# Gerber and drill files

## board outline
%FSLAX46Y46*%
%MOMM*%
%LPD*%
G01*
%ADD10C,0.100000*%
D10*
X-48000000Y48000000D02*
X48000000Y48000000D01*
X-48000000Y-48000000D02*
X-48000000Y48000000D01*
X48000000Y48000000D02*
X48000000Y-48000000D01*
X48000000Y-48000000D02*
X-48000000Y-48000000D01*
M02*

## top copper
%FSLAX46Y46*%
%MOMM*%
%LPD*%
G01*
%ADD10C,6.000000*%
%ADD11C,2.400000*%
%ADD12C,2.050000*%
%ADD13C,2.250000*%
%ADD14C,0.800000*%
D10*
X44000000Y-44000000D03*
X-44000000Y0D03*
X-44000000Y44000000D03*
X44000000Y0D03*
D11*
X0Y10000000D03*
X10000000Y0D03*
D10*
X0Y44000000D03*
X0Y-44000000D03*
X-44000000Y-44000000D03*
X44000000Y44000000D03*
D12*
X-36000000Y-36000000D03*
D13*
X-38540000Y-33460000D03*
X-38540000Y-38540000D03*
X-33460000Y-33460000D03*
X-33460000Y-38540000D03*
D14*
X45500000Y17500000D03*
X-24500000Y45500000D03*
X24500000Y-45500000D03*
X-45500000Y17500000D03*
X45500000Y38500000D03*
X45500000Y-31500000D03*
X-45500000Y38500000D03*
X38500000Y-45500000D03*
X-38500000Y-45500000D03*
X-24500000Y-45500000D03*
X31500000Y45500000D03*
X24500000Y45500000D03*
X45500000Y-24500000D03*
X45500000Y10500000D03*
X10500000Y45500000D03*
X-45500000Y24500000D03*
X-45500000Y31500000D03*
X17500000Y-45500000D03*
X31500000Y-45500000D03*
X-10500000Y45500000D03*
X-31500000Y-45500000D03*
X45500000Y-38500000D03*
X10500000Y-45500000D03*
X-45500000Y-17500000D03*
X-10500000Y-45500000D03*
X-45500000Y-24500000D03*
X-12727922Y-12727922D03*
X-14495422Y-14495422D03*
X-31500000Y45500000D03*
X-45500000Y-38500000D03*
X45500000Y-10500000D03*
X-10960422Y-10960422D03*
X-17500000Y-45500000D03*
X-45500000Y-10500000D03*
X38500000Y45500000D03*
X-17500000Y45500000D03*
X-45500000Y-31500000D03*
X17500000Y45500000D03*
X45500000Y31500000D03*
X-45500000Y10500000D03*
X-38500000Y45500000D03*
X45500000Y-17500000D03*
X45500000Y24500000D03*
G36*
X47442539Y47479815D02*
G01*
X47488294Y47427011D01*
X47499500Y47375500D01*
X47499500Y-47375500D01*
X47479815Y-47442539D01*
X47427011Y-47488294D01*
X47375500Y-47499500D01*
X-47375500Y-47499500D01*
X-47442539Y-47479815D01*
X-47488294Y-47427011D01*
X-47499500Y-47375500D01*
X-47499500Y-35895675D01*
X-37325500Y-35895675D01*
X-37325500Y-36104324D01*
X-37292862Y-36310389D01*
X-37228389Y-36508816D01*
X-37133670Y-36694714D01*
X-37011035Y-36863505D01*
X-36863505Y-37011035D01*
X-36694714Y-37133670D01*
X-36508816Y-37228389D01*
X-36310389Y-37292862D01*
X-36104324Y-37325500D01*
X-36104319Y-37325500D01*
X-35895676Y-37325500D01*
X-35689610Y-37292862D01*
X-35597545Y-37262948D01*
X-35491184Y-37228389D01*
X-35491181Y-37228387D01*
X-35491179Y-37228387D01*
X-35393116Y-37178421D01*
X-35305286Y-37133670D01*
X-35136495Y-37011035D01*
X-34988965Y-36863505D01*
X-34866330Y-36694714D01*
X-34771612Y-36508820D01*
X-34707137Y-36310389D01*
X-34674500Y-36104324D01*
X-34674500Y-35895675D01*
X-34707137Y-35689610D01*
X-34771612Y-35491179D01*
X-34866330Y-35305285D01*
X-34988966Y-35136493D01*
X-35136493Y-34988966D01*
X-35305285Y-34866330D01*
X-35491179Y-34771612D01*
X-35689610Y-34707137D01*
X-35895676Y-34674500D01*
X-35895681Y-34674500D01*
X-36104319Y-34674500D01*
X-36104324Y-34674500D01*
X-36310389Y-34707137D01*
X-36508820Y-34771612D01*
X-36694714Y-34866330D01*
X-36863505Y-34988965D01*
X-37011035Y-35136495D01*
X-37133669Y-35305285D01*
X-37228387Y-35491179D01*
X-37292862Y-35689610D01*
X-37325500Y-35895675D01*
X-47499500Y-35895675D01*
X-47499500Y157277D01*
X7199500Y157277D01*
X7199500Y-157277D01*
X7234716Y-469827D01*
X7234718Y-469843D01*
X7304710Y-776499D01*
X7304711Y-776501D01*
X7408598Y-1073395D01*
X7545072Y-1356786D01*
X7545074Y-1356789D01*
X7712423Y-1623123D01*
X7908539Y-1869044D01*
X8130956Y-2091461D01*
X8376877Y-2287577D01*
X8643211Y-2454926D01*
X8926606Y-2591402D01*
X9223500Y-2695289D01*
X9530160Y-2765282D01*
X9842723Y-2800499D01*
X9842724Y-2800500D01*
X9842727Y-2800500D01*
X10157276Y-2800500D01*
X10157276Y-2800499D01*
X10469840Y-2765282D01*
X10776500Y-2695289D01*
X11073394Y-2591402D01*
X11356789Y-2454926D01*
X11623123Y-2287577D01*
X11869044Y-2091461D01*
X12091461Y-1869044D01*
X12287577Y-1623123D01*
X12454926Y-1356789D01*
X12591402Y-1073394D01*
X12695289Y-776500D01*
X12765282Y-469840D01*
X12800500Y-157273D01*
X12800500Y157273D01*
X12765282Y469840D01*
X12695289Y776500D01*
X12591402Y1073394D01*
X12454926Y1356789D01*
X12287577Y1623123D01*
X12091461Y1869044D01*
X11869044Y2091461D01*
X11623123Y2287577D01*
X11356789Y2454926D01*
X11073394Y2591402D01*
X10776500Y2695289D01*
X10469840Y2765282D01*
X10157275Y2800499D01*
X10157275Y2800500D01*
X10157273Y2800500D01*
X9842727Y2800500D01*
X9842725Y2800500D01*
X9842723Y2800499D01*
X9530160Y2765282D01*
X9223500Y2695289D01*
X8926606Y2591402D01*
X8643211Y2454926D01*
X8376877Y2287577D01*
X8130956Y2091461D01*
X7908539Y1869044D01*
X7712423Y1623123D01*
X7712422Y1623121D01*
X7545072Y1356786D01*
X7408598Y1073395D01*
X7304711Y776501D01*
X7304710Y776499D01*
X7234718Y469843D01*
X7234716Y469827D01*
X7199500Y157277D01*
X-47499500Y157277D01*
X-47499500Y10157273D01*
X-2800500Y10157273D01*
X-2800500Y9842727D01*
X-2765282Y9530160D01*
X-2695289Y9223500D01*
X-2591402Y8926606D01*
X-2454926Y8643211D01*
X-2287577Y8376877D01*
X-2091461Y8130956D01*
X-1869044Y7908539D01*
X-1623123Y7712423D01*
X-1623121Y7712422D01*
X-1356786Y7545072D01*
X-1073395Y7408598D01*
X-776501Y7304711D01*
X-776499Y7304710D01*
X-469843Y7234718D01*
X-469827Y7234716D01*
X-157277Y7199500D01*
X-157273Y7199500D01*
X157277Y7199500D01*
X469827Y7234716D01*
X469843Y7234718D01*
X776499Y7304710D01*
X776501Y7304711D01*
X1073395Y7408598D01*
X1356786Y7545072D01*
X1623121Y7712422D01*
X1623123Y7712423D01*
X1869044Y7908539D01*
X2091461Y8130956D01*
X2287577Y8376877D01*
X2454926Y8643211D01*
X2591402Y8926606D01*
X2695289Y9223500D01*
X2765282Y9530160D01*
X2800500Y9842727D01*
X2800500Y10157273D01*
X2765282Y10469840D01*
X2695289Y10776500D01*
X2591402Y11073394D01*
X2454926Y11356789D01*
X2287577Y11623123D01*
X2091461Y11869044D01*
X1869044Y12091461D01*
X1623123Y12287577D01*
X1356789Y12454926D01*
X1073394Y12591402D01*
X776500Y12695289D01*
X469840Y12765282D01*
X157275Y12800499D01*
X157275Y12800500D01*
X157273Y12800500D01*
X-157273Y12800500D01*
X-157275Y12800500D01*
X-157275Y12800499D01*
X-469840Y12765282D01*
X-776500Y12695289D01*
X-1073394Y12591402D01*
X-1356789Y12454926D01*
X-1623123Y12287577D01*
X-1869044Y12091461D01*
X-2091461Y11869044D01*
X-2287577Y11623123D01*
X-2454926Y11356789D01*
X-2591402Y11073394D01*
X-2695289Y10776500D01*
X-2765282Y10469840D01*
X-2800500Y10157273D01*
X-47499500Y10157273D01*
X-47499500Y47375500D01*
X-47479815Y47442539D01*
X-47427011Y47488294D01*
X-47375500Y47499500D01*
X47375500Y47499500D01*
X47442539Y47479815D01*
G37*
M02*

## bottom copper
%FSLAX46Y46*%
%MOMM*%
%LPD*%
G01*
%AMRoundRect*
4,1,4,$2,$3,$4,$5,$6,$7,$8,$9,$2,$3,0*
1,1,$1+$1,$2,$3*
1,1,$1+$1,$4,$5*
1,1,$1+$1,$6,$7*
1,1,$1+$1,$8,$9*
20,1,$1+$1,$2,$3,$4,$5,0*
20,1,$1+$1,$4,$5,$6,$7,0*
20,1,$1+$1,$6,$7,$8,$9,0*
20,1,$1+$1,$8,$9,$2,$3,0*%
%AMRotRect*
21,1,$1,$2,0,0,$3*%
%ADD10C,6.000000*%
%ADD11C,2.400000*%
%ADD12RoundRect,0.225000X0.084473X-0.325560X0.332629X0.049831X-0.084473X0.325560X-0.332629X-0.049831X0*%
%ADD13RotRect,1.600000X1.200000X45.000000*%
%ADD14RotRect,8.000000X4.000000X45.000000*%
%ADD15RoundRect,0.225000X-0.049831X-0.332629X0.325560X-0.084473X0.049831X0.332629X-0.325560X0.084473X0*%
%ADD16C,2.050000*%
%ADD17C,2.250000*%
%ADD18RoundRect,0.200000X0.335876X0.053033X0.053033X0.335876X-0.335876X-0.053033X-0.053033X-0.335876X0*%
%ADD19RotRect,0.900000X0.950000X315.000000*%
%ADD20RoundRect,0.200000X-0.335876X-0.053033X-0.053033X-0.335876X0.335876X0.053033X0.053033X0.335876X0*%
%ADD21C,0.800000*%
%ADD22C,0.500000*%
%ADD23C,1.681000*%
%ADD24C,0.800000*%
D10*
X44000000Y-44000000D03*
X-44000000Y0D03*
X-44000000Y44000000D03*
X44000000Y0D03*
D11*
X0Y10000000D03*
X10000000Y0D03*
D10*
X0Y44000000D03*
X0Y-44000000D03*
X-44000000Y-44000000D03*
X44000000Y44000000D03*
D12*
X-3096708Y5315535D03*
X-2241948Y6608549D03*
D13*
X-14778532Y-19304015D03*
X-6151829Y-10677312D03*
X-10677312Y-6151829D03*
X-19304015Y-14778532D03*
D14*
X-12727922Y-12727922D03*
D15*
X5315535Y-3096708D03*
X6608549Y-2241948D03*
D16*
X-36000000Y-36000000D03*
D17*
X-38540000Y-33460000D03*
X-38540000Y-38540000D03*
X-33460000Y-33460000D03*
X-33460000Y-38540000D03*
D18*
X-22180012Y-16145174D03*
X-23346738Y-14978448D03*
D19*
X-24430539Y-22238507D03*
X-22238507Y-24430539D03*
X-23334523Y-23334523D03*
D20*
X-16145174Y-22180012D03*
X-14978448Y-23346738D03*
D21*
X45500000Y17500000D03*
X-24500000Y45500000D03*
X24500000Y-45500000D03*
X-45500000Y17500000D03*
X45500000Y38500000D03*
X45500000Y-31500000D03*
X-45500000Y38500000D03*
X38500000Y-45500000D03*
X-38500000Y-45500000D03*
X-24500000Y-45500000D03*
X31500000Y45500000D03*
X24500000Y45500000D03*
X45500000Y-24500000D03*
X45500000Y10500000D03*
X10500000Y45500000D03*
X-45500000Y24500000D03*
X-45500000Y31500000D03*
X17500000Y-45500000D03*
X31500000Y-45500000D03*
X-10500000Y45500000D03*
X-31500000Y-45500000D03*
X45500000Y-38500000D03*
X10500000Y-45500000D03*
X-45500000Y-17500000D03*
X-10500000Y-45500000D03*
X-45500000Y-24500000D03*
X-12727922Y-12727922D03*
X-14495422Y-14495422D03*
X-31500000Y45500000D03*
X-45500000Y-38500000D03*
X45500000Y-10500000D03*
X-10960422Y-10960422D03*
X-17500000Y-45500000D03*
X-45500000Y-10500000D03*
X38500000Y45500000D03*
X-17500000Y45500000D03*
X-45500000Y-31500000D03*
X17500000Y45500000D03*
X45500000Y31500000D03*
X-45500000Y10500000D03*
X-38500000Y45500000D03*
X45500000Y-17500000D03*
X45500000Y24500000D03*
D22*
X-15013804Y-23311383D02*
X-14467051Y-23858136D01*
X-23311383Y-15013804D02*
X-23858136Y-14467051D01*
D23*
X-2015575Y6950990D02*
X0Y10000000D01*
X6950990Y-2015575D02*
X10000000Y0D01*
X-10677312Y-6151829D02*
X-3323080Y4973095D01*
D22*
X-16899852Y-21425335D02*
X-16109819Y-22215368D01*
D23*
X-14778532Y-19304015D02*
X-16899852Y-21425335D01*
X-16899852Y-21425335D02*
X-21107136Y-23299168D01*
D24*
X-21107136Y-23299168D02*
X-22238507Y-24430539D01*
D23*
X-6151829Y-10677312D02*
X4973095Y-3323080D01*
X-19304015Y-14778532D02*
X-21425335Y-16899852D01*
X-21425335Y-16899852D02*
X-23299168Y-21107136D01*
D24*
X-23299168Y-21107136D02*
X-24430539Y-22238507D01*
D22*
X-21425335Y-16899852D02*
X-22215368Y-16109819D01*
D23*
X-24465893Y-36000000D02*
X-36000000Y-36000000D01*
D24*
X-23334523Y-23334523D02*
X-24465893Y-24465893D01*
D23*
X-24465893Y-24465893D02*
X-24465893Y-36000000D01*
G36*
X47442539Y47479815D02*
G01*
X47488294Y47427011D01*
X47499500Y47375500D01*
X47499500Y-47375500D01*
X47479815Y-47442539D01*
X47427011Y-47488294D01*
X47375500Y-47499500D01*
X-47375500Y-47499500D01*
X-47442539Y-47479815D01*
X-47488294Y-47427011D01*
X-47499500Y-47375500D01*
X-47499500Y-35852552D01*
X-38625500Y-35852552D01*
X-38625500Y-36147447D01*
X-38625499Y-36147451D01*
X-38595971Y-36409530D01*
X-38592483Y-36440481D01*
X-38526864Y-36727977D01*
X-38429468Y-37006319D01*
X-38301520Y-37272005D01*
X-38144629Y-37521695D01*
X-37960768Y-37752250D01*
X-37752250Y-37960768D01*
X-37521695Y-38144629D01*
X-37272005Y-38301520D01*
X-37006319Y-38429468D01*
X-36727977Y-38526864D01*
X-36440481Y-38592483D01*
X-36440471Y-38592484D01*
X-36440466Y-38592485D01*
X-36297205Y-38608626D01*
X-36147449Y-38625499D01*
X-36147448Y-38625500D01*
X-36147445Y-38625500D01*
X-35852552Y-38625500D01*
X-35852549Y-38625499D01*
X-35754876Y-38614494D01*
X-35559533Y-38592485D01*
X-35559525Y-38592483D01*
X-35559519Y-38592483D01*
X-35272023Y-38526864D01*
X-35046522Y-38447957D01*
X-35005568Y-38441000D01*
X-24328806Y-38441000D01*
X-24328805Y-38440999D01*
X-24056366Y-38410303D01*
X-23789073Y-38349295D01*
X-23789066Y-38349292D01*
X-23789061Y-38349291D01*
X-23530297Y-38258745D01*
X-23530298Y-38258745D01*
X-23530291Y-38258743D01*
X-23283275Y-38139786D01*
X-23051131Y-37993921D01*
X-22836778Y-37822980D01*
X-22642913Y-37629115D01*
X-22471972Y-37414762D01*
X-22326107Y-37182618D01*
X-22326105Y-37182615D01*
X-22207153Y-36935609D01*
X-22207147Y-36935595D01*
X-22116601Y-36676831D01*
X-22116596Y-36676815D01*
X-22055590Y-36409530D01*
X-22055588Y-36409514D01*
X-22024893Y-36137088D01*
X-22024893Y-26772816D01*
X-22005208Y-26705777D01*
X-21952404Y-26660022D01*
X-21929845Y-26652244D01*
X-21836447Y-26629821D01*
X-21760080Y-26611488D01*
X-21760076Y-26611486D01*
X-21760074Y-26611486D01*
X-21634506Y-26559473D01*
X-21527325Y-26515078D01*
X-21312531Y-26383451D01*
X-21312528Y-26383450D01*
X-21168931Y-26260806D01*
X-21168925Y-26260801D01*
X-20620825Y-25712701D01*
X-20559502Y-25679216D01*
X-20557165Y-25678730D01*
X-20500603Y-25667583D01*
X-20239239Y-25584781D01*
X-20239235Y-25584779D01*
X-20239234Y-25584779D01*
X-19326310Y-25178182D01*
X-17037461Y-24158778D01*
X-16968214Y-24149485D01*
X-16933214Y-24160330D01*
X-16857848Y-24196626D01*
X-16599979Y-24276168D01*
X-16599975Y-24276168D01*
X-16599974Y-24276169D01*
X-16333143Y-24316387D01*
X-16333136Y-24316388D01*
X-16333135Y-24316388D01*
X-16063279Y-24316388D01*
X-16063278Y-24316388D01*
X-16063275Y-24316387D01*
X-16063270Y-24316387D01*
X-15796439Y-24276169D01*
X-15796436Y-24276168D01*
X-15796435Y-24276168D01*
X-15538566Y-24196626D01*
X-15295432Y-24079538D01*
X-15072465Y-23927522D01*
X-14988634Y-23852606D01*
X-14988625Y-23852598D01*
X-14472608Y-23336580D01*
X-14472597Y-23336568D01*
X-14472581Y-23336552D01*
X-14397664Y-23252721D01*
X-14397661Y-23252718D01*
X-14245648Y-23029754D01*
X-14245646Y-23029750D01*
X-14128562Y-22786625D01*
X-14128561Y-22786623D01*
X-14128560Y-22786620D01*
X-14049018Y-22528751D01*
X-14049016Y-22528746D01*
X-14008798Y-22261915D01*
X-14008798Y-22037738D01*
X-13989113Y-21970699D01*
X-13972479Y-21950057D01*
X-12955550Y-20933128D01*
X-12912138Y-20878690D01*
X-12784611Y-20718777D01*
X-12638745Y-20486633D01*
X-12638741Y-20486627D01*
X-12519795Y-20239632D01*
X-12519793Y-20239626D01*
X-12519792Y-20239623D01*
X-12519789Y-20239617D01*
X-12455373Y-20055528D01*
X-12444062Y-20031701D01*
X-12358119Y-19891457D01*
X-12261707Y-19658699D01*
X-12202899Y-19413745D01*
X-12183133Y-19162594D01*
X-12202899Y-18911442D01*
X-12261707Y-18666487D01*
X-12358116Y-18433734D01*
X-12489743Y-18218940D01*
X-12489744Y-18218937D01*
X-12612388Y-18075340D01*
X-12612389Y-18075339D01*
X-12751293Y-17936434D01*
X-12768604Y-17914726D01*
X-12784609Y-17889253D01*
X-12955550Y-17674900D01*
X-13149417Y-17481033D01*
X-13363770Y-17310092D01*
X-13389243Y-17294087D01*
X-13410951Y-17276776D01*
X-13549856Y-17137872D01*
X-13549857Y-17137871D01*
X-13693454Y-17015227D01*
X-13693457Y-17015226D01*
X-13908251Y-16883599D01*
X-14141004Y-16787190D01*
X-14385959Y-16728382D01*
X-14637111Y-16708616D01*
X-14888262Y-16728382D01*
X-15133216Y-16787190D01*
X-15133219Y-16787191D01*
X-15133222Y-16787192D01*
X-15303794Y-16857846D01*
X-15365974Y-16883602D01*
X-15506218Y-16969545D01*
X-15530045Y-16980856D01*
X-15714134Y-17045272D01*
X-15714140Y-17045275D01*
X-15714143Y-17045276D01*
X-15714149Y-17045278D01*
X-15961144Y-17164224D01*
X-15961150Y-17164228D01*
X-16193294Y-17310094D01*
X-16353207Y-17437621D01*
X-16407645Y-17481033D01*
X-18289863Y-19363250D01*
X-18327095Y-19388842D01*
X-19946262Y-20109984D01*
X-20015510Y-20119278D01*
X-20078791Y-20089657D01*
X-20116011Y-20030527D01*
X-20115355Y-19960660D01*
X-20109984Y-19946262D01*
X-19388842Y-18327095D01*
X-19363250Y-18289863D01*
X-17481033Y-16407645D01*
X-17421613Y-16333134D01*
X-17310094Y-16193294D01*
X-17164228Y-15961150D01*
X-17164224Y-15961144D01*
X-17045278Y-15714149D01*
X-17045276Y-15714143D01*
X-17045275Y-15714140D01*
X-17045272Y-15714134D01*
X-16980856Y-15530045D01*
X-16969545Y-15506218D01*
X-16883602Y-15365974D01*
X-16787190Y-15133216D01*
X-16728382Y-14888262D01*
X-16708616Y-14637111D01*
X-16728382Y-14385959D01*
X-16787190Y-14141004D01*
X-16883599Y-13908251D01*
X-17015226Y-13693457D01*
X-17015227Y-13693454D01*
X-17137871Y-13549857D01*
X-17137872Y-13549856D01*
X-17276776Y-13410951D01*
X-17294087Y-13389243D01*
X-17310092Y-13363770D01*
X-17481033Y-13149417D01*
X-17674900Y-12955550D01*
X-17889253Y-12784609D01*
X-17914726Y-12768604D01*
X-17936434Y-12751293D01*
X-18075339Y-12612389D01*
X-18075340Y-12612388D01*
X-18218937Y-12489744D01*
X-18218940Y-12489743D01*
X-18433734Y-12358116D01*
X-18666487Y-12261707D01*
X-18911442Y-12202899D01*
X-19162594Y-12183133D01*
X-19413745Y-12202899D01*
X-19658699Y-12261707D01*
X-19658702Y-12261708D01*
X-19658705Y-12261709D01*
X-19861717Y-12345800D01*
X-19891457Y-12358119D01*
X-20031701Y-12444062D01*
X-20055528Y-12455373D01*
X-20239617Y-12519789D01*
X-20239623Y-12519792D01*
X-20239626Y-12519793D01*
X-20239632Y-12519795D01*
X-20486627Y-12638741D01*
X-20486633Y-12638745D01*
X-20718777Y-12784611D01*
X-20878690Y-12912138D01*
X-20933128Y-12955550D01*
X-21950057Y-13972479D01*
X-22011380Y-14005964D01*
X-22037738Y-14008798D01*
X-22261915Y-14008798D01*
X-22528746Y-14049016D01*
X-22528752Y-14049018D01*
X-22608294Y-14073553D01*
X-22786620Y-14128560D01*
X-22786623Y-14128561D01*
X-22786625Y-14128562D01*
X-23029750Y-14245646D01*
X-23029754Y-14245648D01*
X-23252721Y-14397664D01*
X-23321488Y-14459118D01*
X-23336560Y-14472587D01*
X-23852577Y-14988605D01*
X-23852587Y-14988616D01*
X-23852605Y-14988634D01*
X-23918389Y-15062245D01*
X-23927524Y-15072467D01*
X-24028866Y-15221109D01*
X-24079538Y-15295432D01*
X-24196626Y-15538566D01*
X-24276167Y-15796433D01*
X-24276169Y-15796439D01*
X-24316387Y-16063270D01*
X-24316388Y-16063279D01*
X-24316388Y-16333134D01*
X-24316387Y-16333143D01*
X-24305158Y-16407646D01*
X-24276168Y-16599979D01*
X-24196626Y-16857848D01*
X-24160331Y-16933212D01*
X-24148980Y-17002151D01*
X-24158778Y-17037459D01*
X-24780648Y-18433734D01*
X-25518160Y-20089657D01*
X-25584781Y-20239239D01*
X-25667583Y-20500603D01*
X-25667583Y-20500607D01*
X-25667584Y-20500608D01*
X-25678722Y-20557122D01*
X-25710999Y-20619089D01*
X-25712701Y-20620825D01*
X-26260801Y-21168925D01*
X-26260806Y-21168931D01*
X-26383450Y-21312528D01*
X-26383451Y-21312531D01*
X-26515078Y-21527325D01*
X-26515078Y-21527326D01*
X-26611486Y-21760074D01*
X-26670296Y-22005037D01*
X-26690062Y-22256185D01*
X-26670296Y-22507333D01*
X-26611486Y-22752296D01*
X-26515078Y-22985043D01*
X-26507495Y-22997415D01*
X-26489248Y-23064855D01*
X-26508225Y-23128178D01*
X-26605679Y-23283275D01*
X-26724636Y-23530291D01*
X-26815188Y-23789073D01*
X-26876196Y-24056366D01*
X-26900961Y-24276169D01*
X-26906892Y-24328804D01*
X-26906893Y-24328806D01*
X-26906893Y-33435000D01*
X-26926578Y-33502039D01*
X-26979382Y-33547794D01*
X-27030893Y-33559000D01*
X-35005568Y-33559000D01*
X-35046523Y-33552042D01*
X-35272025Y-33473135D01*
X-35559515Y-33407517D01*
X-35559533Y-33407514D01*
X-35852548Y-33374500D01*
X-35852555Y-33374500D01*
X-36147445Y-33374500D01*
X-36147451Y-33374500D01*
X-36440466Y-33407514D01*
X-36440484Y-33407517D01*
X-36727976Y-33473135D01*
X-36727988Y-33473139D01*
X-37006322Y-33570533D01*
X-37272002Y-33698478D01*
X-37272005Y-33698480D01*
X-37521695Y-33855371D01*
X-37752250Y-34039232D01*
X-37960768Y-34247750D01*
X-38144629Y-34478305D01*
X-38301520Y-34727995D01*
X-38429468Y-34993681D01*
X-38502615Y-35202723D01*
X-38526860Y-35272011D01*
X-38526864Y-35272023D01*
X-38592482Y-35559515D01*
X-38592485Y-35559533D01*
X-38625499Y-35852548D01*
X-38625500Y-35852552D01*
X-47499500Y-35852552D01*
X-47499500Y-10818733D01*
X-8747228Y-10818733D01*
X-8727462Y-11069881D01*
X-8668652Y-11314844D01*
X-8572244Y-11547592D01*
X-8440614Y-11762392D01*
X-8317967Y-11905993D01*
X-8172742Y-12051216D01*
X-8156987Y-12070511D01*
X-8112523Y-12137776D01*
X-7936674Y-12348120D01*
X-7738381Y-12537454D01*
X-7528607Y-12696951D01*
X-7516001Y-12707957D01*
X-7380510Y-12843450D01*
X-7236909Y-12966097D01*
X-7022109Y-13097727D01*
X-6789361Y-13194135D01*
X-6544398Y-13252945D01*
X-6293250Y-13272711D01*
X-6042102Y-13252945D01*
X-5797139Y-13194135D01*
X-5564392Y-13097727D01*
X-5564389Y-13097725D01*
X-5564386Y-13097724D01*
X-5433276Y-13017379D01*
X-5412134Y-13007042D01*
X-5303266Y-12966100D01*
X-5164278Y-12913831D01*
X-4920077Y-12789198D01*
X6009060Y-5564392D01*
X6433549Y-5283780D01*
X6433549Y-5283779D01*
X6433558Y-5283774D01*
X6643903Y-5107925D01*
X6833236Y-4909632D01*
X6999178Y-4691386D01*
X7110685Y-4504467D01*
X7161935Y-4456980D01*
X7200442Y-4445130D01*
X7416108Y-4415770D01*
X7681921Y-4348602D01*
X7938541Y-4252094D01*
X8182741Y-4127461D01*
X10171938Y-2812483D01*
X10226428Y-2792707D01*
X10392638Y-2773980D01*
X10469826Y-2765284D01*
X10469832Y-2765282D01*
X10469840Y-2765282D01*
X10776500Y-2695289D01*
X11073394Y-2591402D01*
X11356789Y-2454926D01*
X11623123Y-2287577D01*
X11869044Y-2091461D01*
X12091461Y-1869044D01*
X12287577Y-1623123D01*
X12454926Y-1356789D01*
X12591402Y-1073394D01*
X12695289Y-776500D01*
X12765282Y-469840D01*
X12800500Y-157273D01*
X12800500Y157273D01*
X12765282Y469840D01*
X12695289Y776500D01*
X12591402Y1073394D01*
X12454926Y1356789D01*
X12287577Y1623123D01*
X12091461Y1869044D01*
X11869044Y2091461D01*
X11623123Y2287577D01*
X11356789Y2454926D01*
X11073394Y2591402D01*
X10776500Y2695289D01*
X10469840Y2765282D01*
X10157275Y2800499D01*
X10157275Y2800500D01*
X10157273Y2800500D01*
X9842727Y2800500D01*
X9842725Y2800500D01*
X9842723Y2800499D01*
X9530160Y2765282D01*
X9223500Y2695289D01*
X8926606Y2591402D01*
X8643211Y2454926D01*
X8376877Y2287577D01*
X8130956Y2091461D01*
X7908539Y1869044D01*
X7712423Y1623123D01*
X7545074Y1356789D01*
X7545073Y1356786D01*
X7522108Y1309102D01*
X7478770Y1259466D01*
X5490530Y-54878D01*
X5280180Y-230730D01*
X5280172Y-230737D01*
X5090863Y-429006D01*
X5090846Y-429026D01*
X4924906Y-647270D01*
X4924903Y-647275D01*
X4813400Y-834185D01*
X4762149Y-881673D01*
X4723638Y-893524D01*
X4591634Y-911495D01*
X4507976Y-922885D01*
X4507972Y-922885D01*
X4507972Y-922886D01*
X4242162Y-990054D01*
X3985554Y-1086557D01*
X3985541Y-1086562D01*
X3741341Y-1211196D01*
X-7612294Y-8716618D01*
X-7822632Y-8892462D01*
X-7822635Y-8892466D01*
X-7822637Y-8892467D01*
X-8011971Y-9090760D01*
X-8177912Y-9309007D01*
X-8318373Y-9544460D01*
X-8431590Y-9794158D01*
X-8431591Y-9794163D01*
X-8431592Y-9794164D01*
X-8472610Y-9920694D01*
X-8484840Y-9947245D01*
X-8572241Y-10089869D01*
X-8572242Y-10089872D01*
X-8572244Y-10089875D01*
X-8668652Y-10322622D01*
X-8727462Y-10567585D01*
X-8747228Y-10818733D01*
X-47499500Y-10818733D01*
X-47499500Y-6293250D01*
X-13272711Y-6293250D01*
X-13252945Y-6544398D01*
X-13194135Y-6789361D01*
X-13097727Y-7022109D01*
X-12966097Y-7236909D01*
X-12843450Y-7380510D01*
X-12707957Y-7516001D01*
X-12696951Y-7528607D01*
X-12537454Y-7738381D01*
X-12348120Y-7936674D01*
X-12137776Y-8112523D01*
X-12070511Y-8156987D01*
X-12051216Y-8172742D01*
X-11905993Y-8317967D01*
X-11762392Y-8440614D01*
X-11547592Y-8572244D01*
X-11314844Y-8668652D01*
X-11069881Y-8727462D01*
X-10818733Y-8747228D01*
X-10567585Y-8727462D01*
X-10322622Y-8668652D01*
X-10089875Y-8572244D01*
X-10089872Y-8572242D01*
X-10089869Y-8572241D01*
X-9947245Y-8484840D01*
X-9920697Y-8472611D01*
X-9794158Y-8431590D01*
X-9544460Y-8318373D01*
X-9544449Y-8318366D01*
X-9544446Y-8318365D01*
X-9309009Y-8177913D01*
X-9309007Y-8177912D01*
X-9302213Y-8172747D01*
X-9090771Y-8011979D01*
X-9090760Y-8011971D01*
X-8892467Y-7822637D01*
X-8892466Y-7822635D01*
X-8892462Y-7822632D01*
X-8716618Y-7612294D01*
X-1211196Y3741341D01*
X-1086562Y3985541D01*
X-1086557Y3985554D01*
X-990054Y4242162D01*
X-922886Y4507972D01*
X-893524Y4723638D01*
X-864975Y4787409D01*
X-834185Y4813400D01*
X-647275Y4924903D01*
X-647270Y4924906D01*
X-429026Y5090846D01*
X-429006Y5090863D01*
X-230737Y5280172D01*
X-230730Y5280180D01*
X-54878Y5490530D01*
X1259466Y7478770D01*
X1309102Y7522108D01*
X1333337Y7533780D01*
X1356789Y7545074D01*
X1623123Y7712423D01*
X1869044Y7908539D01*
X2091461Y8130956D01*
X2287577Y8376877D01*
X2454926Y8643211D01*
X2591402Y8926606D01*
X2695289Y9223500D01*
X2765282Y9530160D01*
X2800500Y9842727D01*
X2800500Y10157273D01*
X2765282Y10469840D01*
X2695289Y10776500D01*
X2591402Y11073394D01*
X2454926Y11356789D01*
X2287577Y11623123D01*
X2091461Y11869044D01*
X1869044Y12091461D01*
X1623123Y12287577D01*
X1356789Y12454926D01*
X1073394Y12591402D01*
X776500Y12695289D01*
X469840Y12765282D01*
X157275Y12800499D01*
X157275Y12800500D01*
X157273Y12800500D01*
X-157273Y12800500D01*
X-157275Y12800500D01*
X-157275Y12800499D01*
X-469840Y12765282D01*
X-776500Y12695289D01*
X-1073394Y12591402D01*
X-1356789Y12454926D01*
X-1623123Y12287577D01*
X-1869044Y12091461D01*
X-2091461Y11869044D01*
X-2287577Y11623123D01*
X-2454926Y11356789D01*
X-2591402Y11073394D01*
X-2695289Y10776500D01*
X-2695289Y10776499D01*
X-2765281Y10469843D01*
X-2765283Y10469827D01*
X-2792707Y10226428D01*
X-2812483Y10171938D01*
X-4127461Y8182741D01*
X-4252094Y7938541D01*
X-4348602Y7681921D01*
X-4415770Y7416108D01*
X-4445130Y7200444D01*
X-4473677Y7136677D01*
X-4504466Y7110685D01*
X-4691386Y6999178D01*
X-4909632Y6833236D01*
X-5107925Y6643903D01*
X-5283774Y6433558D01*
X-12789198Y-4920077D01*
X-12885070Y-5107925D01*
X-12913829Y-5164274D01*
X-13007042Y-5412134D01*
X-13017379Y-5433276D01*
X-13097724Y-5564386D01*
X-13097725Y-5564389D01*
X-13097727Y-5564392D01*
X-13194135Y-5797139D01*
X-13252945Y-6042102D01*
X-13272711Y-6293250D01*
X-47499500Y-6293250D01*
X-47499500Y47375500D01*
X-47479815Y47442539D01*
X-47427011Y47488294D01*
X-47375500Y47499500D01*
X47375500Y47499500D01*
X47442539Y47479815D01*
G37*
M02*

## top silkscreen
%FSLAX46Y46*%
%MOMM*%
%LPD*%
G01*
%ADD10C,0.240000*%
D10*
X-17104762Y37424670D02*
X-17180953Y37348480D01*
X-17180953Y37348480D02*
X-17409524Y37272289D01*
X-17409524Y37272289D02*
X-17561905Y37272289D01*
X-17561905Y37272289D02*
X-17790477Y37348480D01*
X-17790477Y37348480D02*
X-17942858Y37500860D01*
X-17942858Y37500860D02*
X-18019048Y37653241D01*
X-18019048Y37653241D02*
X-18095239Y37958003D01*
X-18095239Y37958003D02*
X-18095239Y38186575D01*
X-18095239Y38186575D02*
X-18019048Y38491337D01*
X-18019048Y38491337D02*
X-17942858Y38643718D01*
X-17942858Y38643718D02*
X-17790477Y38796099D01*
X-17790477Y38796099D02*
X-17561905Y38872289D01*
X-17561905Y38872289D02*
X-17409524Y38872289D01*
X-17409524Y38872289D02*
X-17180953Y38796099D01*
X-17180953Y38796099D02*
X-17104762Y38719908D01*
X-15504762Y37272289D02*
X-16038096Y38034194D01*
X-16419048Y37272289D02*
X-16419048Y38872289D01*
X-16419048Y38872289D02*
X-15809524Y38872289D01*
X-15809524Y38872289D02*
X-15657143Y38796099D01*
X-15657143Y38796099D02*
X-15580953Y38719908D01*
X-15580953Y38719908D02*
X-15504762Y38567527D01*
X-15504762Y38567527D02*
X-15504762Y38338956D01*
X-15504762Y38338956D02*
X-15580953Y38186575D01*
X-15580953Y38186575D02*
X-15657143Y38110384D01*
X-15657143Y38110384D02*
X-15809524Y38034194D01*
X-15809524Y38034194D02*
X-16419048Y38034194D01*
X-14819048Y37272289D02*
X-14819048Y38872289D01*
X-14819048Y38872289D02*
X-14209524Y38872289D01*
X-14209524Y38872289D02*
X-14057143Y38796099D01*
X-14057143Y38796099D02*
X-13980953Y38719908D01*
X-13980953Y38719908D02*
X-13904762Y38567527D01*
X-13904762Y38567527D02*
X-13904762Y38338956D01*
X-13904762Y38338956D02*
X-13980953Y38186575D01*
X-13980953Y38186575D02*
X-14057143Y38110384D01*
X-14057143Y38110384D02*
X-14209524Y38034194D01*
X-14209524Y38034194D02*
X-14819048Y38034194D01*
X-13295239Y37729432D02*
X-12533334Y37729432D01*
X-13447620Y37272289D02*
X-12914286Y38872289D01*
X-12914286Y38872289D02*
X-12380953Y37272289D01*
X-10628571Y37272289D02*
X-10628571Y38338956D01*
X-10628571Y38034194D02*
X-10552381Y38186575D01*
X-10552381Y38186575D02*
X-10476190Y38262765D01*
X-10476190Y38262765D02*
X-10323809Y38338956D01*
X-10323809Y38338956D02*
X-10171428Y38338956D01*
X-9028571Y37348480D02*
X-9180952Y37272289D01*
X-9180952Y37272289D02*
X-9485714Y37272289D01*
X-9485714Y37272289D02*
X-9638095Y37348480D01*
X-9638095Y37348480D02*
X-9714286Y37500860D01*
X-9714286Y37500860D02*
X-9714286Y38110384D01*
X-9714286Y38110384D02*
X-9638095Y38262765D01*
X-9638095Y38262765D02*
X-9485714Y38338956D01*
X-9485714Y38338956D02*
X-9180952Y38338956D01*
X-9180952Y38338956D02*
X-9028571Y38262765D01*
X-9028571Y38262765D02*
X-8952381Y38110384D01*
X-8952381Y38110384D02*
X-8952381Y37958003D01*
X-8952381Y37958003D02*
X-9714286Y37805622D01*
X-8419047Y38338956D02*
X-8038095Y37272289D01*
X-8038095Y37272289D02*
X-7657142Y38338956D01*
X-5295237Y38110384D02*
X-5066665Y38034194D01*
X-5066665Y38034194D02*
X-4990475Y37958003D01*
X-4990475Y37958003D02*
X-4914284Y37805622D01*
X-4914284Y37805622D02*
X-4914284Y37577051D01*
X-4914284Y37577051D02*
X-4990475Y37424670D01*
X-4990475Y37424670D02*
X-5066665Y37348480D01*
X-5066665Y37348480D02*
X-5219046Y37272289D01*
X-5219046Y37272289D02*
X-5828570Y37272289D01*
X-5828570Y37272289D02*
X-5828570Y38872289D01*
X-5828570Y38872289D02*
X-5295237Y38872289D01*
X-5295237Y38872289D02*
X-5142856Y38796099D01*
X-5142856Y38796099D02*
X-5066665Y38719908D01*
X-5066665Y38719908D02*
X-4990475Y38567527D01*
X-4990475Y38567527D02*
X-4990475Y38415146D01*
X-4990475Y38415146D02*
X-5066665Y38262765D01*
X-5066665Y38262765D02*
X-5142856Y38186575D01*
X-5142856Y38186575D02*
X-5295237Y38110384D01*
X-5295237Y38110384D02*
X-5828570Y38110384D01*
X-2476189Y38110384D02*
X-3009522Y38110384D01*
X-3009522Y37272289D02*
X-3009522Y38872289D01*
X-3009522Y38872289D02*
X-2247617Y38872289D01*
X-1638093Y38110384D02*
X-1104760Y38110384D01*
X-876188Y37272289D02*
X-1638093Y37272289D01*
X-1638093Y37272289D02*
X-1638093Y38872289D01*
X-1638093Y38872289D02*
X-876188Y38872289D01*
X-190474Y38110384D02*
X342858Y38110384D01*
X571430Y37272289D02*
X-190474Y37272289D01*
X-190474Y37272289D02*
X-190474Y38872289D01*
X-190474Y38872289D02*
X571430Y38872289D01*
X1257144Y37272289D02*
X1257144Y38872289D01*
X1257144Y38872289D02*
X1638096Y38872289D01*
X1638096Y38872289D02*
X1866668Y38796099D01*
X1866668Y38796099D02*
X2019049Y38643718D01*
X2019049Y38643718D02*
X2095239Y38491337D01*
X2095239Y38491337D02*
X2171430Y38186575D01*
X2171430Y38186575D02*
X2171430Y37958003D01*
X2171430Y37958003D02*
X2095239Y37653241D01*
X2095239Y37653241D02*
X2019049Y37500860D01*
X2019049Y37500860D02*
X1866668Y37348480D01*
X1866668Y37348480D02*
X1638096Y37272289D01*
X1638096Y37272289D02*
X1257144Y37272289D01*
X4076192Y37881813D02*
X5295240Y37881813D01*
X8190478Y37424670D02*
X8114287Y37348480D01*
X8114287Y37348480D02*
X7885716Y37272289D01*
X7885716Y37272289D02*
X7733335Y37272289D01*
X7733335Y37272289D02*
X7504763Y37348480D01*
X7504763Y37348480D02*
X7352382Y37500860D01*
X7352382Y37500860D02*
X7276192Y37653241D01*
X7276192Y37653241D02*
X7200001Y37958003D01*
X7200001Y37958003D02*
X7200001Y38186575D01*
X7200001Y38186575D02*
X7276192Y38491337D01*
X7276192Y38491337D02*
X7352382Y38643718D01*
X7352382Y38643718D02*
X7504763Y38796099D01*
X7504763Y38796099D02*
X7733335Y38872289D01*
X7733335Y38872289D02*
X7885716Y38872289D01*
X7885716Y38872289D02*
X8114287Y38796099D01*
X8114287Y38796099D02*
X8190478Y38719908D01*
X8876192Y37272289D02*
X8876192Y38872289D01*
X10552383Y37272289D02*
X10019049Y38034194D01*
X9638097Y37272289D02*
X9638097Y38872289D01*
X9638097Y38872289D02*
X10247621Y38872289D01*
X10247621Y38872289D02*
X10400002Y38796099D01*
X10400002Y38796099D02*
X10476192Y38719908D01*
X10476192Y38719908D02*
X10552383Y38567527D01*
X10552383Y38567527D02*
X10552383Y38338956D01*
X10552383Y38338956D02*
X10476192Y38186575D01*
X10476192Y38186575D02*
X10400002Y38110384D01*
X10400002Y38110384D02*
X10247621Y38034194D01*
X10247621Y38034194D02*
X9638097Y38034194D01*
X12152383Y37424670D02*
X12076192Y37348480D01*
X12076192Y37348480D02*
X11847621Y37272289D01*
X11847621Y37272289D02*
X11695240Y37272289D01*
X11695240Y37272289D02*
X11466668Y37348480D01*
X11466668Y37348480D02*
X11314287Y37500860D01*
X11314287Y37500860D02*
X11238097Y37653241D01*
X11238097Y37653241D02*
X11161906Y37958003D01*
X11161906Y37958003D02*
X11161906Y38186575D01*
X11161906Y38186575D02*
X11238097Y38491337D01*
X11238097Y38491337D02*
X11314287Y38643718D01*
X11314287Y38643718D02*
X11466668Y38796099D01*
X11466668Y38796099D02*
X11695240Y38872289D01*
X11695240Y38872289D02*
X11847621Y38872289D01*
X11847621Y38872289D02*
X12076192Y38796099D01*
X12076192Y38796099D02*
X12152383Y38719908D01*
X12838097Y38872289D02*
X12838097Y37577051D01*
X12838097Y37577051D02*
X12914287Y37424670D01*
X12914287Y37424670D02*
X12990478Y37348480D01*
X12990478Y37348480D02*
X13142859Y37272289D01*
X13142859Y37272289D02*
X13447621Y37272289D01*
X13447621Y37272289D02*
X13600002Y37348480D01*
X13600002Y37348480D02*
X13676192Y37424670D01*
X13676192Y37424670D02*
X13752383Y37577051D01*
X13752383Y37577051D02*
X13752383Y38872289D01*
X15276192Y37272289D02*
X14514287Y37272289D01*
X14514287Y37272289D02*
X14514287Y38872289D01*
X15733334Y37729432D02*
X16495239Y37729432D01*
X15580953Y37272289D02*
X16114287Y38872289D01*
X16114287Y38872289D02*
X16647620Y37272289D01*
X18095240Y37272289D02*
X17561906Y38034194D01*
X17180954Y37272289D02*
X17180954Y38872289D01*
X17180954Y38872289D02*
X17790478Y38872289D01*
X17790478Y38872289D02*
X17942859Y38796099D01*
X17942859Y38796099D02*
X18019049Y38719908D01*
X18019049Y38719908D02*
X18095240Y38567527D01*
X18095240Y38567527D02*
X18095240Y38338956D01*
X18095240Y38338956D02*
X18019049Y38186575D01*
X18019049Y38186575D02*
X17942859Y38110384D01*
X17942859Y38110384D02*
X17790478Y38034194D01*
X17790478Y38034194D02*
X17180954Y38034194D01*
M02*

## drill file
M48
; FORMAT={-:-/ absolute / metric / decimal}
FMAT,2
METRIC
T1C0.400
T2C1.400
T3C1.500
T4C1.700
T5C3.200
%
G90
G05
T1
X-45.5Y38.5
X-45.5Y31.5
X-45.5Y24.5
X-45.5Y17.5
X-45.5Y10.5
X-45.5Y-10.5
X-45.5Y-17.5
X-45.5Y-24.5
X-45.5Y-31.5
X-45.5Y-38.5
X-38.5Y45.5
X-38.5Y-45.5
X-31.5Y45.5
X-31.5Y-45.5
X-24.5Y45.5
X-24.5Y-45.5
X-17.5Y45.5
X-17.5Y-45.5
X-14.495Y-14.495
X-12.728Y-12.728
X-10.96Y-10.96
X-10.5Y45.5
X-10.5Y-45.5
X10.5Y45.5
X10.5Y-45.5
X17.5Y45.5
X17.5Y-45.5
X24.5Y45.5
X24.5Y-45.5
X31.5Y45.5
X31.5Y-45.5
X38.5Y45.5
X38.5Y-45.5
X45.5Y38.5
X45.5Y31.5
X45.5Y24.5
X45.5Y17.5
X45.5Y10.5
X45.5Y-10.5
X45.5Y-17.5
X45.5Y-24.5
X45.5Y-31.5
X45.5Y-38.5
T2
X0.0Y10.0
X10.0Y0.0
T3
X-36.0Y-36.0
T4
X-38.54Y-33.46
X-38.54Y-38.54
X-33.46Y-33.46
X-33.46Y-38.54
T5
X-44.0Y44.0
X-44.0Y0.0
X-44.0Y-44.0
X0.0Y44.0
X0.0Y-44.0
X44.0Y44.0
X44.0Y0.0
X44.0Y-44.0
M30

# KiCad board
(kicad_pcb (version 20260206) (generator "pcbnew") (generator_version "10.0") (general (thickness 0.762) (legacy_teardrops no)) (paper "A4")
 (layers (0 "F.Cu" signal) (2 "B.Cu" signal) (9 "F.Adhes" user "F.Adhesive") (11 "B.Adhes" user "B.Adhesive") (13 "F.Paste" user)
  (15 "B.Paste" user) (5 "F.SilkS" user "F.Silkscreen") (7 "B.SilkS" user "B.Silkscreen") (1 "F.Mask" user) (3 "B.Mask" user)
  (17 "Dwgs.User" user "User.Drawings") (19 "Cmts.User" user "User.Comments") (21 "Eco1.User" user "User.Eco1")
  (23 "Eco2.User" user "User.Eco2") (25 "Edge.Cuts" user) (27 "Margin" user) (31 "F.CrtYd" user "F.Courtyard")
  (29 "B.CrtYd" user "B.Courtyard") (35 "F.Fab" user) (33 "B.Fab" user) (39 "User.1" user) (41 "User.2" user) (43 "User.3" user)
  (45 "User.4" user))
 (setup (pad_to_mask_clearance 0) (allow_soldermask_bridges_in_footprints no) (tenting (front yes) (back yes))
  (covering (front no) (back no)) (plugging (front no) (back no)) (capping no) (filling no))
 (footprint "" (layer "F.Cu") (at 44 44)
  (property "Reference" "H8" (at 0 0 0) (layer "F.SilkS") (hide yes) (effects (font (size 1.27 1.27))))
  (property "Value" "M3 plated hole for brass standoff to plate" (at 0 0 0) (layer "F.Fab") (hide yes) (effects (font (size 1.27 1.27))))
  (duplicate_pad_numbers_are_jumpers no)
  (pad "1" thru_hole circle (at 0 0) (size 6 6) (drill 3.2) (layers "*.Cu" "*.Mask") (remove_unused_layers no) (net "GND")))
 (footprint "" (layer "F.Cu") (at -44 0)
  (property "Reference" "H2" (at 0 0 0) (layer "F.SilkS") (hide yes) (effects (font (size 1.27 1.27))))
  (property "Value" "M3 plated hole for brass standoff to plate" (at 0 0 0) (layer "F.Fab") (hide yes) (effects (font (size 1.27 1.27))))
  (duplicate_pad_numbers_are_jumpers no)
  (pad "1" thru_hole circle (at 0 0) (size 6 6) (drill 3.2) (layers "*.Cu" "*.Mask") (remove_unused_layers no) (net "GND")))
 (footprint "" (layer "F.Cu") (at -44 -44)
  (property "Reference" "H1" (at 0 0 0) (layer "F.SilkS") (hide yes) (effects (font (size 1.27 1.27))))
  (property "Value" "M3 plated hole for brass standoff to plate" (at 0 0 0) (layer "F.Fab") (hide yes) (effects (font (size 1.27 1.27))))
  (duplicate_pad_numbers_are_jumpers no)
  (pad "1" thru_hole circle (at 0 0) (size 6 6) (drill 3.2) (layers "*.Cu" "*.Mask") (remove_unused_layers no) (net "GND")))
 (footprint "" (layer "F.Cu") (at 44 0)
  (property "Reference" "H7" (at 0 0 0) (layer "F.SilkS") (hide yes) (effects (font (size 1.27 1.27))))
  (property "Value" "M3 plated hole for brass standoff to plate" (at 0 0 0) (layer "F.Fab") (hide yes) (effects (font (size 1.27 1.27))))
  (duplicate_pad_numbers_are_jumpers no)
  (pad "1" thru_hole circle (at 0 0) (size 6 6) (drill 3.2) (layers "*.Cu" "*.Mask") (remove_unused_layers no) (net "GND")))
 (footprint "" (layer "F.Cu") (at 0 -10)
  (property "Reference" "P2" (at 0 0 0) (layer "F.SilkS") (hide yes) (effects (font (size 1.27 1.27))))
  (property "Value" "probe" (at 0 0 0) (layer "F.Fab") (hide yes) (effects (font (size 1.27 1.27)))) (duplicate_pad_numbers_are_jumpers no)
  (pad "1" thru_hole circle (at 0 0) (size 2.4 2.4) (drill 1.4) (layers "*.Cu" "*.Mask") (remove_unused_layers no) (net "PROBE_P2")
   (clearance 1.6)))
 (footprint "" (layer "F.Cu") (at 10 0)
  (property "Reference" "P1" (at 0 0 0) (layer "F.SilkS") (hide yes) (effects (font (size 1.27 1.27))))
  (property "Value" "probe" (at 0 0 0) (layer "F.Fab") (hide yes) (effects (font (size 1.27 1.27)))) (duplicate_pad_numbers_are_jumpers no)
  (pad "1" thru_hole circle (at 0 0) (size 2.4 2.4) (drill 1.4) (layers "*.Cu" "*.Mask") (remove_unused_layers no) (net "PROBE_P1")
   (clearance 1.6)))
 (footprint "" (layer "F.Cu") (at 0 -44)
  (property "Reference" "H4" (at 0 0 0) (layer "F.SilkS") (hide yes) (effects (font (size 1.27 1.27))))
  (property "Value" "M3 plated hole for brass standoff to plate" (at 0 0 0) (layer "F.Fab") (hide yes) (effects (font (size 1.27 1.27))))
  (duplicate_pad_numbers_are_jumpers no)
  (pad "1" thru_hole circle (at 0 0) (size 6 6) (drill 3.2) (layers "*.Cu" "*.Mask") (remove_unused_layers no) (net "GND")))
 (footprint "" (layer "F.Cu") (at 0 44)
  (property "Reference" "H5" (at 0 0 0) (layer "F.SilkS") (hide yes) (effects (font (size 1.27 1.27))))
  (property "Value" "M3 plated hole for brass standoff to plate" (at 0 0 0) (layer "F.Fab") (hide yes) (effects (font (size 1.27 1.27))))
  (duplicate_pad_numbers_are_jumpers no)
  (pad "1" thru_hole circle (at 0 0) (size 6 6) (drill 3.2) (layers "*.Cu" "*.Mask") (remove_unused_layers no) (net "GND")))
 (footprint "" (layer "F.Cu") (at -44 44)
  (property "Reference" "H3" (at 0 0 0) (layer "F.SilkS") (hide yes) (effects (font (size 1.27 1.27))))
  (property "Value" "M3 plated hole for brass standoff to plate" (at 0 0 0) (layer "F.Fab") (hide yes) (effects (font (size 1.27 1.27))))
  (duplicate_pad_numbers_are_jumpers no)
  (pad "1" thru_hole circle (at 0 0) (size 6 6) (drill 3.2) (layers "*.Cu" "*.Mask") (remove_unused_layers no) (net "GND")))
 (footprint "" (layer "F.Cu") (at 44 -44)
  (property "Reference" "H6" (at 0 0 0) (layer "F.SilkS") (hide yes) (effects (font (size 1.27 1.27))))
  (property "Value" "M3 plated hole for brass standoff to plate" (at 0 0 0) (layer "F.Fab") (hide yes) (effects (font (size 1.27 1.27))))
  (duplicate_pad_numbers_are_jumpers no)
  (pad "1" thru_hole circle (at 0 0) (size 6 6) (drill 3.2) (layers "*.Cu" "*.Mask") (remove_unused_layers no) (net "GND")))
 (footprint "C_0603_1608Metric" (layer "B.Cu") (at -2.669328 -5.962042 56.5329438)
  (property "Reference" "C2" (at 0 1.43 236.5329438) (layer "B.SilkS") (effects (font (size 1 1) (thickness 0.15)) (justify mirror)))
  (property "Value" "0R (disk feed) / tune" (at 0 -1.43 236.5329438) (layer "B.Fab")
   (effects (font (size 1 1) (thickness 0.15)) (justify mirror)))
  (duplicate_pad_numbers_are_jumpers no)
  (pad "1" smd roundrect (at -0.775 -0.000001 56.5329438) (size 0.9 0.95) (layers "B.Cu" "B.Mask" "B.Paste") (roundrect_rratio 0.25)
   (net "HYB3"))
  (pad "2" smd roundrect (at 0.775 0.000001 56.5329438) (size 0.9 0.95) (layers "B.Cu" "B.Mask" "B.Paste") (roundrect_rratio 0.25)
   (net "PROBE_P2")))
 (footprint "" (layer "B.Cu") (at -12.727922 12.727922 45)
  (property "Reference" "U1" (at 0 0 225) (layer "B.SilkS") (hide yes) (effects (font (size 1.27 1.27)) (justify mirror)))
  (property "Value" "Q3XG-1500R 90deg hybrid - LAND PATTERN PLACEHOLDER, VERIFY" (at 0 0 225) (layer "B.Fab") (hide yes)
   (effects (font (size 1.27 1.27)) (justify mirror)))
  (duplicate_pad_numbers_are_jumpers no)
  (pad "1" smd rect (at -6.1 3.2 45) (size 1.6 1.2) (layers "B.Cu" "B.Mask" "B.Paste") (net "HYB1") (thermal_bridge_angle 45))
  (pad "2" smd rect (at 6.1 3.2 45) (size 1.6 1.2) (layers "B.Cu" "B.Mask" "B.Paste") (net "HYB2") (thermal_bridge_angle 45))
  (pad "3" smd rect (at 6.1 -3.2 45) (size 1.6 1.2) (layers "B.Cu" "B.Mask" "B.Paste") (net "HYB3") (thermal_bridge_angle 45))
  (pad "4" smd rect (at -6.1 -3.2 45) (size 1.6 1.2) (layers "B.Cu" "B.Mask" "B.Paste") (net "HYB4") (thermal_bridge_angle 45))
  (pad "5" smd rect (at 0 0 45) (size 8 4) (layers "B.Cu" "B.Mask" "B.Paste") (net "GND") (thermal_bridge_angle 45)))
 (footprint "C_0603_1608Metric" (layer "B.Cu") (at 5.962042 2.669328 33.4670562)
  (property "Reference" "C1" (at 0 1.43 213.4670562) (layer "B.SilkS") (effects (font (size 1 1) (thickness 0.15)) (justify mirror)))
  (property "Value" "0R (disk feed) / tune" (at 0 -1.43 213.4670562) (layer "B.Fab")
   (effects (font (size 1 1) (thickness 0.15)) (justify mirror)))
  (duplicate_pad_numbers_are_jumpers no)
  (pad "1" smd roundrect (at -0.775 0.000001 33.4670562) (size 0.9 0.95) (layers "B.Cu" "B.Mask" "B.Paste") (roundrect_rratio 0.25)
   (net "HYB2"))
  (pad "2" smd roundrect (at 0.775 -0.000001 33.4670562) (size 0.9 0.95) (layers "B.Cu" "B.Mask" "B.Paste") (roundrect_rratio 0.25)
   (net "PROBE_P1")))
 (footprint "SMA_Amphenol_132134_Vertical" (layer "B.Cu") (at -36 36)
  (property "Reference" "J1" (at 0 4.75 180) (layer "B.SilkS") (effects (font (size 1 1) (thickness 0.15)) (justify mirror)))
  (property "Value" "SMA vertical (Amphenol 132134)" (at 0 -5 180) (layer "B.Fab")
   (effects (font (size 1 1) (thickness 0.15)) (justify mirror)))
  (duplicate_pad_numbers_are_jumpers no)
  (pad "1" thru_hole circle (at 0 0) (size 2.05 2.05) (drill 1.5) (layers "*.Cu" "*.Mask") (remove_unused_layers no) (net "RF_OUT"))
  (pad "2" thru_hole circle (at -2.54 -2.54) (size 2.25 2.25) (drill 1.7) (layers "*.Cu" "*.Mask") (remove_unused_layers no) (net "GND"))
  (pad "2" thru_hole circle (at -2.54 2.54) (size 2.25 2.25) (drill 1.7) (layers "*.Cu" "*.Mask") (remove_unused_layers no) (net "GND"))
  (pad "2" thru_hole circle (at 2.54 -2.54) (size 2.25 2.25) (drill 1.7) (layers "*.Cu" "*.Mask") (remove_unused_layers no) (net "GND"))
  (pad "2" thru_hole circle (at 2.54 2.54) (size 2.25 2.25) (drill 1.7) (layers "*.Cu" "*.Mask") (remove_unused_layers no) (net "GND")))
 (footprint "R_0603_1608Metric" (layer "B.Cu") (at -22.763375 15.561811 135)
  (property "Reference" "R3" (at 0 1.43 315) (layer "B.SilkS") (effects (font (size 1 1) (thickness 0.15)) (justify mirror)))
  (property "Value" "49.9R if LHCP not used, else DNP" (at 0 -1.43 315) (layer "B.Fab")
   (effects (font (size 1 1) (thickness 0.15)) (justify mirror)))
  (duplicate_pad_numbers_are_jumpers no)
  (pad "1" smd roundrect (at -0.825 0 135) (size 0.8 0.95) (layers "B.Cu" "B.Mask" "B.Paste") (roundrect_rratio 0.25) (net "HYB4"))
  (pad "2" smd roundrect (at 0.825 0 135) (size 0.8 0.95) (layers "B.Cu" "B.Mask" "B.Paste") (roundrect_rratio 0.25) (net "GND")))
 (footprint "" (layer "B.Cu") (at -23.334523 23.334523 -45)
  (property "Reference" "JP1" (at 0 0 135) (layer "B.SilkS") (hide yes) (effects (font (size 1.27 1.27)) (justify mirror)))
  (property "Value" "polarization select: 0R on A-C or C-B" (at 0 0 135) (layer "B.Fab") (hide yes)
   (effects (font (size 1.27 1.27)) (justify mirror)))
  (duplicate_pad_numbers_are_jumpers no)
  (pad "A" smd rect (at -1.550001 0 315) (size 0.9 0.95) (layers "B.Cu" "B.Mask" "B.Paste") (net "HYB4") (thermal_bridge_angle 45))
  (pad "B" smd rect (at 1.550001 0 315) (size 0.9 0.95) (layers "B.Cu" "B.Mask" "B.Paste") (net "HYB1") (thermal_bridge_angle 45))
  (pad "C" smd rect (at 0 0 315) (size 0.9 0.95) (layers "B.Cu" "B.Mask" "B.Paste") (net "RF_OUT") (thermal_bridge_angle 45)))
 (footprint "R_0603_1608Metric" (layer "B.Cu") (at -15.561811 22.763375 -45)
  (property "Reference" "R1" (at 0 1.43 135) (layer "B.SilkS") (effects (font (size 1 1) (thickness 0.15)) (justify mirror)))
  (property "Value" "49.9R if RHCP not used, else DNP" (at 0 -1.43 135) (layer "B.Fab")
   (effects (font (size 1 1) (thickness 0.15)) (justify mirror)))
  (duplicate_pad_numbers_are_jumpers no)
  (pad "1" smd roundrect (at -0.825 0 315) (size 0.8 0.95) (layers "B.Cu" "B.Mask" "B.Paste") (roundrect_rratio 0.25) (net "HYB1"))
  (pad "2" smd roundrect (at 0.825 0 315) (size 0.8 0.95) (layers "B.Cu" "B.Mask" "B.Paste") (roundrect_rratio 0.25) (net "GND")))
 (gr_line (start -48 -48) (end 48 -48) (stroke (width 0.1) (type default)) (layer "Edge.Cuts"))
 (gr_line (start -48 48) (end -48 -48) (stroke (width 0.1) (type default)) (layer "Edge.Cuts"))
 (gr_line (start 48 -48) (end 48 48) (stroke (width 0.1) (type default)) (layer "Edge.Cuts"))
 (gr_line (start 48 48) (end -48 48) (stroke (width 0.1) (type default)) (layer "Edge.Cuts"))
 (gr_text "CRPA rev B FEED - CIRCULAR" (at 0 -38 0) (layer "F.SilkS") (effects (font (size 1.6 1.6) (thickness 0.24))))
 (via (at 45.5 -17.5) (size 0.8) (drill 0.4) (layers "F.Cu" "B.Cu") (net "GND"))
 (via (at -24.5 -45.5) (size 0.8) (drill 0.4) (layers "F.Cu" "B.Cu") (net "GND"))
 (via (at 24.5 45.5) (size 0.8) (drill 0.4) (layers "F.Cu" "B.Cu") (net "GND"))
 (via (at -45.5 -17.5) (size 0.8) (drill 0.4) (layers "F.Cu" "B.Cu") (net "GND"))
 (via (at 45.5 -38.5) (size 0.8) (drill 0.4) (layers "F.Cu" "B.Cu") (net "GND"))
 (via (at 45.5 31.5) (size 0.8) (drill 0.4) (layers "F.Cu" "B.Cu") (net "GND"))
 (via (at -45.5 -38.5) (size 0.8) (drill 0.4) (layers "F.Cu" "B.Cu") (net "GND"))
 (via (at 38.5 45.5) (size 0.8) (drill 0.4) (layers "F.Cu" "B.Cu") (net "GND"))
 (via (at -38.5 45.5) (size 0.8) (drill 0.4) (layers "F.Cu" "B.Cu") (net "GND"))
 (via (at -24.5 45.5) (size 0.8) (drill 0.4) (layers "F.Cu" "B.Cu") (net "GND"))
 (via (at 31.5 -45.5) (size 0.8) (drill 0.4) (layers "F.Cu" "B.Cu") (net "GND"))
 (via (at 24.5 -45.5) (size 0.8) (drill 0.4) (layers "F.Cu" "B.Cu") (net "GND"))
 (via (at 45.5 24.5) (size 0.8) (drill 0.4) (layers "F.Cu" "B.Cu") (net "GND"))
 (via (at 45.5 -10.5) (size 0.8) (drill 0.4) (layers "F.Cu" "B.Cu") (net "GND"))
 (via (at 10.5 -45.5) (size 0.8) (drill 0.4) (layers "F.Cu" "B.Cu") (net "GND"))
 (via (at -45.5 -24.5) (size 0.8) (drill 0.4) (layers "F.Cu" "B.Cu") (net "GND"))
 (via (at -45.5 -31.5) (size 0.8) (drill 0.4) (layers "F.Cu" "B.Cu") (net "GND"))
 (via (at 17.5 45.5) (size 0.8) (drill 0.4) (layers "F.Cu" "B.Cu") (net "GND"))
 (via (at 31.5 45.5) (size 0.8) (drill 0.4) (layers "F.Cu" "B.Cu") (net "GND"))
 (via (at -10.5 -45.5) (size 0.8) (drill 0.4) (layers "F.Cu" "B.Cu") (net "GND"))
 (via (at -31.5 45.5) (size 0.8) (drill 0.4) (layers "F.Cu" "B.Cu") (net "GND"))
 (via (at 45.5 38.5) (size 0.8) (drill 0.4) (layers "F.Cu" "B.Cu") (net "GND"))
 (via (at 10.5 45.5) (size 0.8) (drill 0.4) (layers "F.Cu" "B.Cu") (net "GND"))
 (via (at -45.5 17.5) (size 0.8) (drill 0.4) (layers "F.Cu" "B.Cu") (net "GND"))
 (via (at -10.5 45.5) (size 0.8) (drill 0.4) (layers "F.Cu" "B.Cu") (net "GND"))
 (via (at -45.5 24.5) (size 0.8) (drill 0.4) (layers "F.Cu" "B.Cu") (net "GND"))
 (via (at -12.727922 12.727922) (size 0.8) (drill 0.4) (layers "F.Cu" "B.Cu") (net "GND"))
 (via (at -14.495422 14.495422) (size 0.8) (drill 0.4) (layers "F.Cu" "B.Cu") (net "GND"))
 (via (at -31.5 -45.5) (size 0.8) (drill 0.4) (layers "F.Cu" "B.Cu") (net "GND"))
 (via (at -45.5 38.5) (size 0.8) (drill 0.4) (layers "F.Cu" "B.Cu") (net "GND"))
 (via (at 45.5 10.5) (size 0.8) (drill 0.4) (layers "F.Cu" "B.Cu") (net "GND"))
 (via (at -10.960422 10.960422) (size 0.8) (drill 0.4) (layers "F.Cu" "B.Cu") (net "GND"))
 (via (at -17.5 45.5) (size 0.8) (drill 0.4) (layers "F.Cu" "B.Cu") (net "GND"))
 (via (at -45.5 10.5) (size 0.8) (drill 0.4) (layers "F.Cu" "B.Cu") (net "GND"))
 (via (at 38.5 -45.5) (size 0.8) (drill 0.4) (layers "F.Cu" "B.Cu") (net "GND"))
 (via (at -17.5 -45.5) (size 0.8) (drill 0.4) (layers "F.Cu" "B.Cu") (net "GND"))
 (via (at -45.5 31.5) (size 0.8) (drill 0.4) (layers "F.Cu" "B.Cu") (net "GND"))
 (via (at 17.5 -45.5) (size 0.8) (drill 0.4) (layers "F.Cu" "B.Cu") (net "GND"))
 (via (at 45.5 -31.5) (size 0.8) (drill 0.4) (layers "F.Cu" "B.Cu") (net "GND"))
 (via (at -45.5 -10.5) (size 0.8) (drill 0.4) (layers "F.Cu" "B.Cu") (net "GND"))
 (via (at -38.5 -45.5) (size 0.8) (drill 0.4) (layers "F.Cu" "B.Cu") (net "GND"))
 (via (at 45.5 17.5) (size 0.8) (drill 0.4) (layers "F.Cu" "B.Cu") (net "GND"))
 (via (at 45.5 -24.5) (size 0.8) (drill 0.4) (layers "F.Cu" "B.Cu") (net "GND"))
 (segment (start -15.013804 23.311383) (end -14.467051 23.858136) (width 0.5) (layer "B.Cu") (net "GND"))
 (segment (start -23.311383 15.013804) (end -23.858136 14.467051) (width 0.5) (layer "B.Cu") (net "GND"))
 (segment (start -2.015575 -6.95099) (end 0 -10) (width 1.681) (layer "B.Cu") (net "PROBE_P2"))
 (segment (start 6.95099 2.015575) (end 10 0) (width 1.681) (layer "B.Cu") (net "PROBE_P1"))
 (segment (start -10.677312 6.151829) (end -3.32308 -4.973095) (width 1.681) (layer "B.Cu") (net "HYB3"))
 (segment (start -16.899852 21.425335) (end -16.109819 22.215368) (width 0.5) (layer "B.Cu") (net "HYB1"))
 (segment (start -14.778532 19.304015) (end -16.899852 21.425335) (width 1.681) (layer "B.Cu") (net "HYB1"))
 (segment (start -16.899852 21.425335) (end -21.107136 23.299168) (width 1.681) (layer "B.Cu") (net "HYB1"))
 (segment (start -21.107136 23.299168) (end -22.238507 24.430539) (width 0.8) (layer "B.Cu") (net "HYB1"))
 (segment (start -6.151829 10.677312) (end 4.973095 3.32308) (width 1.681) (layer "B.Cu") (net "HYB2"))
 (segment (start -19.304015 14.778532) (end -21.425335 16.899852) (width 1.681) (layer "B.Cu") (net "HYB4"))
 (segment (start -21.425335 16.899852) (end -23.299168 21.107136) (width 1.681) (layer "B.Cu") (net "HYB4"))
 (segment (start -23.299168 21.107136) (end -24.430539 22.238507) (width 0.8) (layer "B.Cu") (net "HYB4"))
 (segment (start -21.425335 16.899852) (end -22.215368 16.109819) (width 0.5) (layer "B.Cu") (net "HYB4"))
 (segment (start -24.465893 36) (end -36 36) (width 1.681) (layer "B.Cu") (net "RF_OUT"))
 (segment (start -23.334523 23.334523) (end -24.465893 24.465893) (width 0.8) (layer "B.Cu") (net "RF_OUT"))
 (segment (start -24.465893 24.465893) (end -24.465893 36) (width 1.681) (layer "B.Cu") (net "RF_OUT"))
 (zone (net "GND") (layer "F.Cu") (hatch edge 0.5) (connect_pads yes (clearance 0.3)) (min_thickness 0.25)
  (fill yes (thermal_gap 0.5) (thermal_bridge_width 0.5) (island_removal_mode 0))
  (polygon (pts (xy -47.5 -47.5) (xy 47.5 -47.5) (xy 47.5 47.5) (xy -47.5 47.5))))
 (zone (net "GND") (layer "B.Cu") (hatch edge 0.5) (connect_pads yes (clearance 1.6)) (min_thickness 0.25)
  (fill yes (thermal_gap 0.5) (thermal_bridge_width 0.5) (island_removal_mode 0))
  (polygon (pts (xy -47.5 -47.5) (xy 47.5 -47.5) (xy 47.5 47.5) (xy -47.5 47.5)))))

